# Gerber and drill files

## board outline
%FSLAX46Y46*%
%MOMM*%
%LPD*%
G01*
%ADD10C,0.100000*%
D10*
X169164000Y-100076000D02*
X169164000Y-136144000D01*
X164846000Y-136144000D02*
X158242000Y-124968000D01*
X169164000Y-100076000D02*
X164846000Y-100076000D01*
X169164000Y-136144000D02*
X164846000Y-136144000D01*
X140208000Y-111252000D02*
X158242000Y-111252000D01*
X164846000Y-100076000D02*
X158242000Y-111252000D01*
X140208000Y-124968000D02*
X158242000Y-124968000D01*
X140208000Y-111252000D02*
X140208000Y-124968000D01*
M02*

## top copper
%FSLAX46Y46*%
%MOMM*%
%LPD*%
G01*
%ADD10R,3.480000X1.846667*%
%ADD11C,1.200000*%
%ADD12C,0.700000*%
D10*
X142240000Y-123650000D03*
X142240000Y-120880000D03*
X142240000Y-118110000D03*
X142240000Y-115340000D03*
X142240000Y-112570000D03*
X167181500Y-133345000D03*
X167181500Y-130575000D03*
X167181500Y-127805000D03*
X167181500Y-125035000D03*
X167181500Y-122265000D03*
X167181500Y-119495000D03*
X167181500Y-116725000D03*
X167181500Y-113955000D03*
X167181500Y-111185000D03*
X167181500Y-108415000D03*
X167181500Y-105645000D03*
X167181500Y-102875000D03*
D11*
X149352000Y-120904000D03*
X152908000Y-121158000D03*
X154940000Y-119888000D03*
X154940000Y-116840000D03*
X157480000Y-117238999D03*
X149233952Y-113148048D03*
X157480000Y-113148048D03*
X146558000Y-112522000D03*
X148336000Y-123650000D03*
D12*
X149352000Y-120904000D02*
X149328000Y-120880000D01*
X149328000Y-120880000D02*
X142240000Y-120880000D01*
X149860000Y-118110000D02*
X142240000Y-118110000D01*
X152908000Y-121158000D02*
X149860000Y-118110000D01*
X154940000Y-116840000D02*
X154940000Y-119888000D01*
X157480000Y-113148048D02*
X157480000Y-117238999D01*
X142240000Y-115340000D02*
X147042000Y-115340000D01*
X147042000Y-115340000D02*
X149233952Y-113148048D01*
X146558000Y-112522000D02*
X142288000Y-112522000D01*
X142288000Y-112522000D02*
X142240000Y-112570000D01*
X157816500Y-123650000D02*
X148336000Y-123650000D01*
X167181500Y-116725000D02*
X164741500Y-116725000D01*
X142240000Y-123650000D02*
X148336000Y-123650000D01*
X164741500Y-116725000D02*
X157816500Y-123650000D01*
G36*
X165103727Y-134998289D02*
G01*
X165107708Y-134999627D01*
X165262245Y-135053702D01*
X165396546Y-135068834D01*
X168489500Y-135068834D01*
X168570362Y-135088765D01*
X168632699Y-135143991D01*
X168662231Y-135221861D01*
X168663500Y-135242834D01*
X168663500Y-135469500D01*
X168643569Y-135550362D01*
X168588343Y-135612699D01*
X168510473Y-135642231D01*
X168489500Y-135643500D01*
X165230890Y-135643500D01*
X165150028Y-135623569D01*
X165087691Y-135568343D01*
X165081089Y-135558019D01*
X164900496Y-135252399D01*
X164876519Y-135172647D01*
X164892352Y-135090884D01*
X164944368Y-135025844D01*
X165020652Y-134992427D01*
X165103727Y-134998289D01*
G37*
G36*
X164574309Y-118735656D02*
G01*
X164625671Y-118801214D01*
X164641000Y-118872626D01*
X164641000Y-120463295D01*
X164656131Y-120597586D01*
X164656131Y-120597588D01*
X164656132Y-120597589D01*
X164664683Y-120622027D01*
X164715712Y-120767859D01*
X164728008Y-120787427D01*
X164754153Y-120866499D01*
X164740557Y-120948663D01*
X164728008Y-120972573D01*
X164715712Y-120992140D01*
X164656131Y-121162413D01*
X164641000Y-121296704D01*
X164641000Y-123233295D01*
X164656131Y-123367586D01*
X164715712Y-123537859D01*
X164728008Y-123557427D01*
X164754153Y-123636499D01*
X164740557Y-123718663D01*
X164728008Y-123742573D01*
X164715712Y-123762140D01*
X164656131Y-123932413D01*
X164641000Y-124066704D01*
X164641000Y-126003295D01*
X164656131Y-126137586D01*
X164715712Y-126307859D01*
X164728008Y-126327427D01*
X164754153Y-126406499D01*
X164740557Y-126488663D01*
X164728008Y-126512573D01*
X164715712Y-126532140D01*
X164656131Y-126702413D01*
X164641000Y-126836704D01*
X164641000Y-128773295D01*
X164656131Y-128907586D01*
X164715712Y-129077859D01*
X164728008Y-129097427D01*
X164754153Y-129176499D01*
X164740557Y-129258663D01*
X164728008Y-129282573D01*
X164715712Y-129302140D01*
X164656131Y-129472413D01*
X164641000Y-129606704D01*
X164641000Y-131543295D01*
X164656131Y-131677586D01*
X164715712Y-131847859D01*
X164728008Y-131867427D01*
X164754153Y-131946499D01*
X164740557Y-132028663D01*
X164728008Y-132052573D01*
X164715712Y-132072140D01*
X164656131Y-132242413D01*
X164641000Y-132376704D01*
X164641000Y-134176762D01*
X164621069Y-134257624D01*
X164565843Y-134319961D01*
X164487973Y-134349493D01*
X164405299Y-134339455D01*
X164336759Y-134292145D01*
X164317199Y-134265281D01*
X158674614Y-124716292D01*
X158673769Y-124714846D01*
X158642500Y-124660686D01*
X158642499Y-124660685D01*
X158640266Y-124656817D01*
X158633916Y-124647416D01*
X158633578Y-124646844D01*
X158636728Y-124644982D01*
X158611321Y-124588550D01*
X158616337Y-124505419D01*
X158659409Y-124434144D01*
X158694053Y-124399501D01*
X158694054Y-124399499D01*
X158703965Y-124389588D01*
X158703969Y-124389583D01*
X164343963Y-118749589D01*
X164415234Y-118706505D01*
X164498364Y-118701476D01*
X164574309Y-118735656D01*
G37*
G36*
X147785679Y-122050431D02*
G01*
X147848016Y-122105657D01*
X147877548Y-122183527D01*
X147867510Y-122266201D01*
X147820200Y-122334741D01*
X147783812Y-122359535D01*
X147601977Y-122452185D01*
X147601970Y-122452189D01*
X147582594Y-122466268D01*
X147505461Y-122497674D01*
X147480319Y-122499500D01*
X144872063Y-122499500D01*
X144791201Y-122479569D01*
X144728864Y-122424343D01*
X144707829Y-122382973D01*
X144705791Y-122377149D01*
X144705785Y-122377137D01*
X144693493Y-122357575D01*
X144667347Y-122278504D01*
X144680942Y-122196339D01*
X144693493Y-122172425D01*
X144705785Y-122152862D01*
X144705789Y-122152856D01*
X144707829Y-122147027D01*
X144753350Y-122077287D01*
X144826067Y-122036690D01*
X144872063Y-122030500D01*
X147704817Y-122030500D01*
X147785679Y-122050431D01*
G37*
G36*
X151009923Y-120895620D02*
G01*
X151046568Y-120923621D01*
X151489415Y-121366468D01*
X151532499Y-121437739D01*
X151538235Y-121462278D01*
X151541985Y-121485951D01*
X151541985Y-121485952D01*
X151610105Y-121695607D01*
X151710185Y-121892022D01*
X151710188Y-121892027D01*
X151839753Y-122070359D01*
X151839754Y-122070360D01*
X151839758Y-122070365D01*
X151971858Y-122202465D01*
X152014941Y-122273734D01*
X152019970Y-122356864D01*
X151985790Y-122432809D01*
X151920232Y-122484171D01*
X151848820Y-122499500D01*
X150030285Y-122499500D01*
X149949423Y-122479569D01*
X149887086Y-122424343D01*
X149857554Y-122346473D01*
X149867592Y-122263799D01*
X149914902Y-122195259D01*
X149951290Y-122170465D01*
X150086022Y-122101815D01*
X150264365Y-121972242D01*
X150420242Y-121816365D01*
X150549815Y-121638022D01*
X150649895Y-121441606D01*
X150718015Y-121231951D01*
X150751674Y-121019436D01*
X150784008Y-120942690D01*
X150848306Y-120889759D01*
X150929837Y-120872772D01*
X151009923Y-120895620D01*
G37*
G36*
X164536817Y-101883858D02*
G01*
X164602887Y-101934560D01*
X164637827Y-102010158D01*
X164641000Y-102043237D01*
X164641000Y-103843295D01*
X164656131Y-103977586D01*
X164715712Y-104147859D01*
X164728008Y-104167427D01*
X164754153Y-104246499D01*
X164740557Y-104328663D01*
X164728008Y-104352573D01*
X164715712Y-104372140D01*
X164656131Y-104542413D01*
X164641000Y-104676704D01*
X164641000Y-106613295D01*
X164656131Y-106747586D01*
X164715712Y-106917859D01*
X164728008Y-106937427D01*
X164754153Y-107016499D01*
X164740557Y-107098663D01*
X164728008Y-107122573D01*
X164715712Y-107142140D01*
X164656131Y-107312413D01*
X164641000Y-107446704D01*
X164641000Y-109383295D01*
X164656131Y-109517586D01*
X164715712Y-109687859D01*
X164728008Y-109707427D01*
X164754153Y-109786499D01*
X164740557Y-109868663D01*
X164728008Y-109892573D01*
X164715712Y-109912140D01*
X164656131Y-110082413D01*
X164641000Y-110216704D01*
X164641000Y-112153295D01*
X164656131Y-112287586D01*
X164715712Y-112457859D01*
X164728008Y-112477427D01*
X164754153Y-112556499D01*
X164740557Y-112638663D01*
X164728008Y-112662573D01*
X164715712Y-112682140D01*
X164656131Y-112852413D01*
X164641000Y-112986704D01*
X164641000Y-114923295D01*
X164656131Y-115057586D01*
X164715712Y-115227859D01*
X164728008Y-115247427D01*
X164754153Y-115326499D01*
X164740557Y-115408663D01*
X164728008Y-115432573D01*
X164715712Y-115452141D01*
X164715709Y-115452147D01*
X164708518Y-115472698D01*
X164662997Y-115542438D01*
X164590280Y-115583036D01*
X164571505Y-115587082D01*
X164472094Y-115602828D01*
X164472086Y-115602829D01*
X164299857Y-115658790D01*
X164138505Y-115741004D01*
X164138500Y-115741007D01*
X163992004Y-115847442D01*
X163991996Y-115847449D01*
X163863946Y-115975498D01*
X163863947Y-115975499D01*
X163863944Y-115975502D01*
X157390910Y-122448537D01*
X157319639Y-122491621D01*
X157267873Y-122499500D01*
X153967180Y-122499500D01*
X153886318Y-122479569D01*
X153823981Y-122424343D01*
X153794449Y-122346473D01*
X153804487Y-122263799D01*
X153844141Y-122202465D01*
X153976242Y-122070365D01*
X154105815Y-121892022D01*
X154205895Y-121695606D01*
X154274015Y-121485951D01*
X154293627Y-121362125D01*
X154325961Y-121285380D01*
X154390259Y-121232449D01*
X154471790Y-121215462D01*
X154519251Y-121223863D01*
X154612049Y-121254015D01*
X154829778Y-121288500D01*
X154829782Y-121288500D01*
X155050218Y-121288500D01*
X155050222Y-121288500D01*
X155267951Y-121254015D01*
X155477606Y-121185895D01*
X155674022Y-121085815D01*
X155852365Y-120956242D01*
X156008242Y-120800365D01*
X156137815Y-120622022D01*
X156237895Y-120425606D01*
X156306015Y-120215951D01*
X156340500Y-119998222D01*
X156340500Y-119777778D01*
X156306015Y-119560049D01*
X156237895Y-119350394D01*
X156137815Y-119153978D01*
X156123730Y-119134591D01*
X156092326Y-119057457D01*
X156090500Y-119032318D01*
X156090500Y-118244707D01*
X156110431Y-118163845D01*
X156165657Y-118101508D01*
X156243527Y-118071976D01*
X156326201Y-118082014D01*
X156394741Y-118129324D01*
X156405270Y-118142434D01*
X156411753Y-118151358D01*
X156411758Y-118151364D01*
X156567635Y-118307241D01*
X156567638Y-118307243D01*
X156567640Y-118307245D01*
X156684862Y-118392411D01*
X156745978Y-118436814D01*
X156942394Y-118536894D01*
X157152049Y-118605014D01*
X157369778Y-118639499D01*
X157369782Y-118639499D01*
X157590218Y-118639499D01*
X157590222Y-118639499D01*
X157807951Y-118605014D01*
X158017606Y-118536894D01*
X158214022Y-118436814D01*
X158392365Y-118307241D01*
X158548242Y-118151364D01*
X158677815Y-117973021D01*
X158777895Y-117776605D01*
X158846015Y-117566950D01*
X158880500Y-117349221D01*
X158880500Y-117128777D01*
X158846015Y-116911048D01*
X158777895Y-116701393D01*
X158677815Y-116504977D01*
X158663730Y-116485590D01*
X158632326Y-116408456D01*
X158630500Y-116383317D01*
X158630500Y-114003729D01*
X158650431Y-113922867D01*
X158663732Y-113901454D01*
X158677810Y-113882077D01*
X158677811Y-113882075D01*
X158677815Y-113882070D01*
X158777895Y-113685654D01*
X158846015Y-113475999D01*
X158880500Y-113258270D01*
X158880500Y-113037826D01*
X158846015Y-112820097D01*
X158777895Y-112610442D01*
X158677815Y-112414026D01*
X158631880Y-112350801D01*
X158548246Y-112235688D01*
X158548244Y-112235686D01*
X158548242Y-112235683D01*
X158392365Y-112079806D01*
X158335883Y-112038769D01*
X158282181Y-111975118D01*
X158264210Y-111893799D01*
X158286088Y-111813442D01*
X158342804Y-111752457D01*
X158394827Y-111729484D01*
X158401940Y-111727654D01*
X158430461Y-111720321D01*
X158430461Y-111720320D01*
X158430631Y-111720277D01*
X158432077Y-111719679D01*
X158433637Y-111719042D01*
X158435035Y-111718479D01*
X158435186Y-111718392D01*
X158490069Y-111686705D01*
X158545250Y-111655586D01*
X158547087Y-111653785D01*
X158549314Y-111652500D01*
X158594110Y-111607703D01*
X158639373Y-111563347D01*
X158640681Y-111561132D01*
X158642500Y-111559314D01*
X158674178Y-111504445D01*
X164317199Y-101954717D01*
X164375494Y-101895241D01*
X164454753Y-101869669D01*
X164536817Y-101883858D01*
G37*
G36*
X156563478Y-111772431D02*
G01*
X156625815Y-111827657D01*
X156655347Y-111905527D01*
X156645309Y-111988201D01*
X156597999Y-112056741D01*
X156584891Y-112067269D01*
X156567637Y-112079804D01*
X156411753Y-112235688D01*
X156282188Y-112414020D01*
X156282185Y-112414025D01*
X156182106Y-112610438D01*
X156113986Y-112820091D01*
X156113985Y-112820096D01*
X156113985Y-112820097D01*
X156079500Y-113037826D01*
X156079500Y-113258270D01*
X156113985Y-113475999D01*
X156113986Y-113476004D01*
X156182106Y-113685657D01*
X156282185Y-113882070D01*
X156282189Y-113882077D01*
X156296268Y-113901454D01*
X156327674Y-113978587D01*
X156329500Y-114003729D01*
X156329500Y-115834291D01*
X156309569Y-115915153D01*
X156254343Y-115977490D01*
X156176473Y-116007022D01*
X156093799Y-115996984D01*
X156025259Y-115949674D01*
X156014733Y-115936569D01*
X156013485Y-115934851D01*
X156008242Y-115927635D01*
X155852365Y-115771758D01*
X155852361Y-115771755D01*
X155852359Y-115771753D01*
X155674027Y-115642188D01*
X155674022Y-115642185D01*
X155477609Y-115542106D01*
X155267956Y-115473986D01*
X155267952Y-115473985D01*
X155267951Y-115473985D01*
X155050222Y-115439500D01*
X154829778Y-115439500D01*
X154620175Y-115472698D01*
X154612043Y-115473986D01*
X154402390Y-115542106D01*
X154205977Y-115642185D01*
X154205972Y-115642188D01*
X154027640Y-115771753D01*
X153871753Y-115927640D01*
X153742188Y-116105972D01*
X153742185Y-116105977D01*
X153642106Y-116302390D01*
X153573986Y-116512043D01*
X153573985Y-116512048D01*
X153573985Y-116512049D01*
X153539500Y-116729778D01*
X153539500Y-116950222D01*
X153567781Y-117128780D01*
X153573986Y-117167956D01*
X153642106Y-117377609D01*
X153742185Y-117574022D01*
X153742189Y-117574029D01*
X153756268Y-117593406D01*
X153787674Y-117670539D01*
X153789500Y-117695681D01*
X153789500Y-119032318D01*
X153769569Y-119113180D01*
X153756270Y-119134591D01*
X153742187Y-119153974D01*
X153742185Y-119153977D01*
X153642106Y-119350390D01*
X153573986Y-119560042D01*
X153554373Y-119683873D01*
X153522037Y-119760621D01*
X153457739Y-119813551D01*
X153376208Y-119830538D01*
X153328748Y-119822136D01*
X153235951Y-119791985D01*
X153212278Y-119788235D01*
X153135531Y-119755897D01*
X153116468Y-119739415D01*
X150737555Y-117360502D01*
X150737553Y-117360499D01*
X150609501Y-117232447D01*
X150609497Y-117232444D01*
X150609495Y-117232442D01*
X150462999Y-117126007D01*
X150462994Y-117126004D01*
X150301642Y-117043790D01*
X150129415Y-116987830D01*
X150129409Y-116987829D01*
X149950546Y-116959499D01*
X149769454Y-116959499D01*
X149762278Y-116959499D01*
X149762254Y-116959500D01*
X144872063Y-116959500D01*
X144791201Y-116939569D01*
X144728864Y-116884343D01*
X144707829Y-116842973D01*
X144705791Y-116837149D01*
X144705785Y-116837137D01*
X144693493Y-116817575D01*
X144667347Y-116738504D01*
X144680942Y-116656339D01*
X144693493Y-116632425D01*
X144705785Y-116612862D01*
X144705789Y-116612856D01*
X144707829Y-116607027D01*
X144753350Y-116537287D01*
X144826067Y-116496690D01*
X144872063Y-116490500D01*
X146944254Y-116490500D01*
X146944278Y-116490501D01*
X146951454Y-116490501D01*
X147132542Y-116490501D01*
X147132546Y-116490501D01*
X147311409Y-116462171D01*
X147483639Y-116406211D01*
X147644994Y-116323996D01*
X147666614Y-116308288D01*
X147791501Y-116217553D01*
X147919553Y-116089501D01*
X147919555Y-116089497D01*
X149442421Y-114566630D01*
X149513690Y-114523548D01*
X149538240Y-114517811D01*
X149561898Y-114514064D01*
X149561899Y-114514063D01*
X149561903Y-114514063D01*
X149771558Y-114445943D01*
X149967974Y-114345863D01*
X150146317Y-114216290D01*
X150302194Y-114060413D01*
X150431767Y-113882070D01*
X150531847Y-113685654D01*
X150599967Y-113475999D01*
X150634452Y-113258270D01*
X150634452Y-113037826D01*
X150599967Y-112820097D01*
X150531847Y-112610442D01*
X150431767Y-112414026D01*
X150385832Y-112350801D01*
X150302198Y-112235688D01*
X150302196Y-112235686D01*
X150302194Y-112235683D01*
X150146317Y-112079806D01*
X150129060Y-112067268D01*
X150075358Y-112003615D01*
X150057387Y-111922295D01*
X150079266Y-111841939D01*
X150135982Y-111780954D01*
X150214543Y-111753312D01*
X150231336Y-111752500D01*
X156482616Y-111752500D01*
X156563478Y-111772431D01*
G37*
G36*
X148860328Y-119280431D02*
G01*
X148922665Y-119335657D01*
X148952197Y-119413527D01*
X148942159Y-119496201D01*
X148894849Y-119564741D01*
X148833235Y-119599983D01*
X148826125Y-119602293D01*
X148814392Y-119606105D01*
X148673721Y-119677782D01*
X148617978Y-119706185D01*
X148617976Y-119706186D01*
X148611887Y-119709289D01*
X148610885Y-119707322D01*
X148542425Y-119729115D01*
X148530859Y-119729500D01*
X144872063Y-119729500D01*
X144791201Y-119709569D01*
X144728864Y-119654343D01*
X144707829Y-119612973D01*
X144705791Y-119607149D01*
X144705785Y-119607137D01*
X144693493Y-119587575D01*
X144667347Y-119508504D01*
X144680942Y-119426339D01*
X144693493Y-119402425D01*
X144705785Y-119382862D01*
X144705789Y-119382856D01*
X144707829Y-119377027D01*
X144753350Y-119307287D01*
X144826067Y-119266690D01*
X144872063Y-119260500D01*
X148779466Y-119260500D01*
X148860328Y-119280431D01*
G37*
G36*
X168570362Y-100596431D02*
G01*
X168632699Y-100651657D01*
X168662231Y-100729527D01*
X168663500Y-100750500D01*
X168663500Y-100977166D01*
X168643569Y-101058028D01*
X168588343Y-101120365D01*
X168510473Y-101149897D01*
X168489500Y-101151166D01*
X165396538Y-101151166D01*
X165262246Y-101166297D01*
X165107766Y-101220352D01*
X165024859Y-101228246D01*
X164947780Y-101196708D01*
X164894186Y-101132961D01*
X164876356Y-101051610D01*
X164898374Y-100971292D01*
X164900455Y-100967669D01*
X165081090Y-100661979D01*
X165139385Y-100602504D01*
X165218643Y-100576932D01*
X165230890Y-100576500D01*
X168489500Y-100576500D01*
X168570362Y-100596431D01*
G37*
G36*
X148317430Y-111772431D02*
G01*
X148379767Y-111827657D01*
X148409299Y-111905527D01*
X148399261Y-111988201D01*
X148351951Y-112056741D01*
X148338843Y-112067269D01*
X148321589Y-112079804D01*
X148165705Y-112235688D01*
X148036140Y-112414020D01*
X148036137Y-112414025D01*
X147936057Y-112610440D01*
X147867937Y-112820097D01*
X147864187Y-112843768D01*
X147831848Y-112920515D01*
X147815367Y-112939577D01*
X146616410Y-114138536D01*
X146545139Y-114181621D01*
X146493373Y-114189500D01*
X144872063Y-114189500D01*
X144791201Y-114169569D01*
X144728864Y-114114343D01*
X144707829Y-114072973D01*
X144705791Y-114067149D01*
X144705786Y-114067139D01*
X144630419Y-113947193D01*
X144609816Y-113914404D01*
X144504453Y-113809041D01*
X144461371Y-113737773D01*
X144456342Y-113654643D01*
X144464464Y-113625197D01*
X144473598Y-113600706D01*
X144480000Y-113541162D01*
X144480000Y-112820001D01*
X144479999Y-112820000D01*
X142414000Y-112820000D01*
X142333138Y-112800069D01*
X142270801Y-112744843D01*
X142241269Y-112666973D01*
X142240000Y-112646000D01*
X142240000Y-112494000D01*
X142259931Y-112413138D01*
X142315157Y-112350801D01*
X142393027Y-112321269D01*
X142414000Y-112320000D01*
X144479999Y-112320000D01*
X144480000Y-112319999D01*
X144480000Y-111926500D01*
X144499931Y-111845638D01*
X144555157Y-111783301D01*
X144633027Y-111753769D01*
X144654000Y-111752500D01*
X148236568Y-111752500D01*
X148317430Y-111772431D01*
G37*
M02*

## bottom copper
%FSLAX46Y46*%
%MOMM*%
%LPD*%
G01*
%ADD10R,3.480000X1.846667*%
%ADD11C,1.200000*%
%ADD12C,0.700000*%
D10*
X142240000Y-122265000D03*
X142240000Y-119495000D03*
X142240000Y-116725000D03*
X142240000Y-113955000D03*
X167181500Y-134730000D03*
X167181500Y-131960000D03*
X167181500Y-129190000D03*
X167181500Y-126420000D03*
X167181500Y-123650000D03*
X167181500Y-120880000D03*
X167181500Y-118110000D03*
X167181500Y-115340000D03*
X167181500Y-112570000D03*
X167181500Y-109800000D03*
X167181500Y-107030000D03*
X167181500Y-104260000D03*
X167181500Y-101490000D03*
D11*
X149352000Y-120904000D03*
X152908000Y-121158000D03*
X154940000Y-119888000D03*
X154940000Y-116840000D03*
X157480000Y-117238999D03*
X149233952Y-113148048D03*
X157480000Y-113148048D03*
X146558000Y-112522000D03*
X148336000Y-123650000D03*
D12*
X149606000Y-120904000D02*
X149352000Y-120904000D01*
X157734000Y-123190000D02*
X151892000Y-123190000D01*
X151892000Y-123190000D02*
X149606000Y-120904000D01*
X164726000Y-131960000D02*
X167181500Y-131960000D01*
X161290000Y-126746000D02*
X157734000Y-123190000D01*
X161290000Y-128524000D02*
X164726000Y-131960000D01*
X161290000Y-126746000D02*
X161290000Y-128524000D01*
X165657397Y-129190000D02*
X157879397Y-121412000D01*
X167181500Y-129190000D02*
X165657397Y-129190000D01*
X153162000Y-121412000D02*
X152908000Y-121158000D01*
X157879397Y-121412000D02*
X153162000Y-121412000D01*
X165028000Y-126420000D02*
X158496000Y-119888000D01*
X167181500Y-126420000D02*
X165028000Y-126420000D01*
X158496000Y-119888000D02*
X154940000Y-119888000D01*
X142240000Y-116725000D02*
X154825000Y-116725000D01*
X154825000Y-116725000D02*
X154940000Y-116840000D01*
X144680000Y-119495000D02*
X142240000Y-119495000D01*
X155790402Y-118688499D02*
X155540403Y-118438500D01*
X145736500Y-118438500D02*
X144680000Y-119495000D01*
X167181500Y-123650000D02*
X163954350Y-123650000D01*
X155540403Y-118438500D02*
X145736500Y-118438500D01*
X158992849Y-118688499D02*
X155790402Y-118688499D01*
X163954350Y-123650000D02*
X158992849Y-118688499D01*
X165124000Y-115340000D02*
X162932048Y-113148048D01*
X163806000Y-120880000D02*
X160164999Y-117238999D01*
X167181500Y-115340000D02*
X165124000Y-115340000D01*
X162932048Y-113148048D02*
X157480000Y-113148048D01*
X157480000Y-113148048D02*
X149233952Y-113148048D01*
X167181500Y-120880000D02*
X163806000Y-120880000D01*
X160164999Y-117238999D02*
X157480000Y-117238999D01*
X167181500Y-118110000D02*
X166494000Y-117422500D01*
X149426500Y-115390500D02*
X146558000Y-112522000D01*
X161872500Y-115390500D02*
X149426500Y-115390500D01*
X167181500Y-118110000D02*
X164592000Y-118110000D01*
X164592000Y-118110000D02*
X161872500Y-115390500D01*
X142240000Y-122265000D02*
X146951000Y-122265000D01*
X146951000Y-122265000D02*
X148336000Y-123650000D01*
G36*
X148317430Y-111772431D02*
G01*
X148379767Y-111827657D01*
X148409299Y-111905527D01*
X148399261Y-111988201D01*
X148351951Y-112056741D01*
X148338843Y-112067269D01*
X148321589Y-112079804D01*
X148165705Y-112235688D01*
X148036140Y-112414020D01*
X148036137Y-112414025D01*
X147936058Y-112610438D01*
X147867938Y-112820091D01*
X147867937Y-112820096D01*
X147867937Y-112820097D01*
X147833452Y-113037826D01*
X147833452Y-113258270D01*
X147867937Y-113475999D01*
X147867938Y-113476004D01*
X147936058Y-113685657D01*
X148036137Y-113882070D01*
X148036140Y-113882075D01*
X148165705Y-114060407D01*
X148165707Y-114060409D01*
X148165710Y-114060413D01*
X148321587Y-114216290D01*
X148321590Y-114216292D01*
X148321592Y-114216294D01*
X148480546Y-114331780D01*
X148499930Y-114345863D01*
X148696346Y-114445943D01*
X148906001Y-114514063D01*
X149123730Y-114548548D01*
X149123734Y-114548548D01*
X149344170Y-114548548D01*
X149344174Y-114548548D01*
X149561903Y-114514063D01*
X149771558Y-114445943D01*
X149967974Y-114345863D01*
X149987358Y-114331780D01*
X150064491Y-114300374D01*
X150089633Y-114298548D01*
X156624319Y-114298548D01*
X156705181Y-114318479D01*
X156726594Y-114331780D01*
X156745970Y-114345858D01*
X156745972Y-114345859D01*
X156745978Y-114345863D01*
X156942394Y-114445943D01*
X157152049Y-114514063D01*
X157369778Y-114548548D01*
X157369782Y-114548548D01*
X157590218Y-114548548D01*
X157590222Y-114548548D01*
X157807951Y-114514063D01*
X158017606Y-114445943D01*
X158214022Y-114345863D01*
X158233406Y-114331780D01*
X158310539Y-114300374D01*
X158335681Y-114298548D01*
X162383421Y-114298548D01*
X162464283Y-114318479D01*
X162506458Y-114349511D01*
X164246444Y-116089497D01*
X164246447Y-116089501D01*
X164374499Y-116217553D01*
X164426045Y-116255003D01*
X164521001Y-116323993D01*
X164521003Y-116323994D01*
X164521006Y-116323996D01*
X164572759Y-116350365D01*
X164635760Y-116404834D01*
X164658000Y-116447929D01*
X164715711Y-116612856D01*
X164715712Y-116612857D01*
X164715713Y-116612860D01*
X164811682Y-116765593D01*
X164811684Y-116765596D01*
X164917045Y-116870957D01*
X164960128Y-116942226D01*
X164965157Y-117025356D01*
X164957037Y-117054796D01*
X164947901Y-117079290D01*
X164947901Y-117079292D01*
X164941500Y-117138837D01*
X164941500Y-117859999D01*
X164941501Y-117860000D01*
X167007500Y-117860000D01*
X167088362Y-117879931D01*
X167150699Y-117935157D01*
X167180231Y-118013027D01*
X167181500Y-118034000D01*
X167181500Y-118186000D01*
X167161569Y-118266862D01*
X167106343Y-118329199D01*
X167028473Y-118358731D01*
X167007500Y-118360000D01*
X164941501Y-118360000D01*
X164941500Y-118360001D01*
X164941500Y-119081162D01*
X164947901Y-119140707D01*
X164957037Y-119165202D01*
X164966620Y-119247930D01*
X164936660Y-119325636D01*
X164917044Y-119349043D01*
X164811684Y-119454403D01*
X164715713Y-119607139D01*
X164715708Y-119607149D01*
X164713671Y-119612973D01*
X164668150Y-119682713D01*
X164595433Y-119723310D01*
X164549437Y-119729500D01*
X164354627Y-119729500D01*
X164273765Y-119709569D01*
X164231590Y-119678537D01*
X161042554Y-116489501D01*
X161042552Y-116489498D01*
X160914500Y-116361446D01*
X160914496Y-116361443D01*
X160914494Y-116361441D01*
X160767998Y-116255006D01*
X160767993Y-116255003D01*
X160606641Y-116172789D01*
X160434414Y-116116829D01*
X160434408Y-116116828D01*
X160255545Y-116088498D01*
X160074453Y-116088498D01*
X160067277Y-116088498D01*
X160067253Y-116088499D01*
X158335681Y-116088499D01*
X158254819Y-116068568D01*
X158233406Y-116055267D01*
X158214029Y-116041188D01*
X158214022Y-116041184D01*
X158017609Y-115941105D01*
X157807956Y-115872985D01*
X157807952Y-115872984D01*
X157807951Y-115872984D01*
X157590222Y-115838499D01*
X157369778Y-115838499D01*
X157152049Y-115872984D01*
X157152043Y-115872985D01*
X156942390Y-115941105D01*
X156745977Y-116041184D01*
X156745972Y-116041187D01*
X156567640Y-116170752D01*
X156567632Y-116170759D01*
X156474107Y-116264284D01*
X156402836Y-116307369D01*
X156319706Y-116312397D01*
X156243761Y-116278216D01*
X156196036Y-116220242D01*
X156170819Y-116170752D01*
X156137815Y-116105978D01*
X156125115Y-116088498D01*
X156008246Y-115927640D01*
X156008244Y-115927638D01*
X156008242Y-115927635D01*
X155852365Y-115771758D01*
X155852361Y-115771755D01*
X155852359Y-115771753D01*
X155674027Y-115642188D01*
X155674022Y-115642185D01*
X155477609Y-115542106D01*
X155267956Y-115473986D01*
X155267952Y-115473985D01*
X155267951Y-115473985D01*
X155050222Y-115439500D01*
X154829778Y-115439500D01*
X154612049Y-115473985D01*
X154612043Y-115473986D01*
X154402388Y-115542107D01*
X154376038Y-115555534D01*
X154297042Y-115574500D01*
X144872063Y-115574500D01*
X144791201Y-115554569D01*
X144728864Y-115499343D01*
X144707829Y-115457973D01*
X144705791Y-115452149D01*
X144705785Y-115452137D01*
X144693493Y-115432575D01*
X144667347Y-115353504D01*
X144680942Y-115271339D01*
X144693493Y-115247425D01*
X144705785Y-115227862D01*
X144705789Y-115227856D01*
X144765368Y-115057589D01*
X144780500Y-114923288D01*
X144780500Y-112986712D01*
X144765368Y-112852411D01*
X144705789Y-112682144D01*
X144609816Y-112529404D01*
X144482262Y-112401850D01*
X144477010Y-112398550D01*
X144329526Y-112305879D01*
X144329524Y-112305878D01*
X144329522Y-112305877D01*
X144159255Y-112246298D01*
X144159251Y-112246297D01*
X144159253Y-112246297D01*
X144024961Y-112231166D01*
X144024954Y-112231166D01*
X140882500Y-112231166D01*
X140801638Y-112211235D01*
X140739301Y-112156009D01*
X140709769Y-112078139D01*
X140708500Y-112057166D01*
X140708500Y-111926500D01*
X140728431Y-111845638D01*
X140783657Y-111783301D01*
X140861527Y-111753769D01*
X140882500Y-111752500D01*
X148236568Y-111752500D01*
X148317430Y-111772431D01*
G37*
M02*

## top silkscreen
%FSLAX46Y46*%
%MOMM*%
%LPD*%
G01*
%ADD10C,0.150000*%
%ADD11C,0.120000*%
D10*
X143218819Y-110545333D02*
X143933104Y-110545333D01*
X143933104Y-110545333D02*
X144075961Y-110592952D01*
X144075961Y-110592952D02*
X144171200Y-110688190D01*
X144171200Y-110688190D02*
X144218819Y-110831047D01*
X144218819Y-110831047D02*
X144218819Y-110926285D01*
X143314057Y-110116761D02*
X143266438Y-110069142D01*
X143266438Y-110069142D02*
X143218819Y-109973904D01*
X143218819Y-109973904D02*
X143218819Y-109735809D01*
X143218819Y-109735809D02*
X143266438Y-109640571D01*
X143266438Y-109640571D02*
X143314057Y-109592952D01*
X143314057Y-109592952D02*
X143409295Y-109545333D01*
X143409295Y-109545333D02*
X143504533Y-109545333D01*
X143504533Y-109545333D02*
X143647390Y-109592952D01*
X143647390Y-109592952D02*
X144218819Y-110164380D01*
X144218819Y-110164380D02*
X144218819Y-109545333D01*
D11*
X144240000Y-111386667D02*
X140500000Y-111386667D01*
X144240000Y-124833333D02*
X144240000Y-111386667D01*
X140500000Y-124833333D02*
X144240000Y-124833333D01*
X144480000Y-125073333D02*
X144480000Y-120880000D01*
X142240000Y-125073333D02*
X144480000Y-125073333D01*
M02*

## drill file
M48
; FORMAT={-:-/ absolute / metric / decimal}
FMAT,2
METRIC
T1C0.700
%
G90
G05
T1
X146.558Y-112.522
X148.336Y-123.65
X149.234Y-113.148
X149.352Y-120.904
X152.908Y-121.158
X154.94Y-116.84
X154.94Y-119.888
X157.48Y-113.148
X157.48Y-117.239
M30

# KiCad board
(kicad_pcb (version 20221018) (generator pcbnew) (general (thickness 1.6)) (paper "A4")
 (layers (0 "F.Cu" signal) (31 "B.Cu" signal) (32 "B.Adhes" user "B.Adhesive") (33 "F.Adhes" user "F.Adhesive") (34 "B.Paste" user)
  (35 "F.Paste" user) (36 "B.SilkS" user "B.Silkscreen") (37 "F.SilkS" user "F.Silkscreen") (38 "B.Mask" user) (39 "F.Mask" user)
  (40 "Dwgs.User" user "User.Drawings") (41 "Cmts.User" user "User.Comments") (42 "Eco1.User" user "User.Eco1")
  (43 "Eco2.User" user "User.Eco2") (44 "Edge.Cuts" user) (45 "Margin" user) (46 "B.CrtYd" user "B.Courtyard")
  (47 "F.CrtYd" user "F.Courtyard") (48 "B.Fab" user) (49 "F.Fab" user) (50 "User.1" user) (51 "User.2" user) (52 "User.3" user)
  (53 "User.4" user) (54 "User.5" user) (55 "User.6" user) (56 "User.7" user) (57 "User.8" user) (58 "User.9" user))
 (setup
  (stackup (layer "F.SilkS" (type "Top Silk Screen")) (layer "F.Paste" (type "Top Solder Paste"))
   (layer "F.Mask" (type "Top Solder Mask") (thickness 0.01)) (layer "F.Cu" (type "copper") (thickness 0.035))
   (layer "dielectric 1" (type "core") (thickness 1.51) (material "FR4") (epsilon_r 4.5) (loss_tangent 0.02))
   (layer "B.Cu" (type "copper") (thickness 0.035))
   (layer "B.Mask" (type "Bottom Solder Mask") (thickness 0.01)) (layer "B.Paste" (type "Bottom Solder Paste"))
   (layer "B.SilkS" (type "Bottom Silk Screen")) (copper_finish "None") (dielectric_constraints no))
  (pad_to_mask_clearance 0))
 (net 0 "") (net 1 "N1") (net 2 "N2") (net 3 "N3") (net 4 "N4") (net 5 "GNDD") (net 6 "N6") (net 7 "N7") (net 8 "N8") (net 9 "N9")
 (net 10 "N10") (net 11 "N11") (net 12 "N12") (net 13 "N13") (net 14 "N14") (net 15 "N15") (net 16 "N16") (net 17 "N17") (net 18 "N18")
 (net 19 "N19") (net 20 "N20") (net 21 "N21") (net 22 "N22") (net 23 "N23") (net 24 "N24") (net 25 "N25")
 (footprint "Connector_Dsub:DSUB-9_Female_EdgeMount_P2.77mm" (layer "F.Cu") (at 142.24 118.11 -90)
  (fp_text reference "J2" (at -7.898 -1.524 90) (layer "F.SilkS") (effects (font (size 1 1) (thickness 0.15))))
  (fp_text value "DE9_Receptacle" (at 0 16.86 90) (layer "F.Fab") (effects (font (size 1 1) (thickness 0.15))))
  (fp_line (start -6.723333 -2) (end -6.723333 1.74) (stroke (width 0.12) (type solid)) (layer "F.SilkS"))
  (fp_line (start 6.723333 -2) (end -6.723333 -2) (stroke (width 0.12) (type solid)) (layer "F.SilkS"))
  (fp_line (start 6.723333 1.74) (end 6.723333 -2) (stroke (width 0.12) (type solid)) (layer "F.SilkS"))
  (fp_line (start 6.963333 -2.24) (end 2.77 -2.24) (stroke (width 0.12) (type solid)) (layer "F.SilkS"))
  (fp_line (start 6.963333 0) (end 6.963333 -2.24) (stroke (width 0.12) (type solid)) (layer "F.SilkS"))
  (pad "1" smd rect (at 5.54 0 270) (size 1.846667 3.48) (layers "F.Cu" "F.Paste" "F.Mask") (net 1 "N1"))
  (pad "2" smd rect (at 2.77 0 270) (size 1.846667 3.48) (layers "F.Cu" "F.Paste" "F.Mask") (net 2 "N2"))
  (pad "3" smd rect (at 0 0 270) (size 1.846667 3.48) (layers "F.Cu" "F.Paste" "F.Mask") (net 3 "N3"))
  (pad "4" smd rect (at -2.77 0 270) (size 1.846667 3.48) (layers "F.Cu" "F.Paste" "F.Mask") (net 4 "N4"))
  (pad "5" smd rect (at -5.54 0 270) (size 1.846667 3.48) (layers "F.Cu" "F.Paste" "F.Mask") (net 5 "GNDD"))
  (pad "6" smd rect (at 4.155 0 270) (size 1.846667 3.48) (layers "B.Cu" "B.Paste" "B.Mask") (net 1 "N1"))
  (pad "7" smd rect (at 1.385 0 270) (size 1.846667 3.48) (layers "B.Cu" "B.Paste" "B.Mask") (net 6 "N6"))
  (pad "8" smd rect (at -1.385 0 270) (size 1.846667 3.48) (layers "B.Cu" "B.Paste" "B.Mask") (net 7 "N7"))
  (pad "9" smd rect (at -4.155 0 270) (size 1.846667 3.48) (layers "B.Cu" "B.Paste" "B.Mask") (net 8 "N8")))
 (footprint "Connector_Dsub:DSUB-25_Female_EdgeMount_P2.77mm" (layer "B.Cu") (at 167.1815 118.11 -90)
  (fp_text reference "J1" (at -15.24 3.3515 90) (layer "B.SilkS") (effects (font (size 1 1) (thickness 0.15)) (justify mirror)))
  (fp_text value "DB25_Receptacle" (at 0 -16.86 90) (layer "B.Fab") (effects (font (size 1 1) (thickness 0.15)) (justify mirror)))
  (pad "1" smd rect (at 16.62 0 270) (size 1.846667 3.48) (layers "B.Cu" "B.Paste" "B.Mask") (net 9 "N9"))
  (pad "2" smd rect (at 13.85 0 270) (size 1.846667 3.48) (layers "B.Cu" "B.Paste" "B.Mask") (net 2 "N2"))
  (pad "3" smd rect (at 11.08 0 270) (size 1.846667 3.48) (layers "B.Cu" "B.Paste" "B.Mask") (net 3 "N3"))
  (pad "4" smd rect (at 8.31 0 270) (size 1.846667 3.48) (layers "B.Cu" "B.Paste" "B.Mask") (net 7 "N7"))
  (pad "5" smd rect (at 5.54 0 270) (size 1.846667 3.48) (layers "B.Cu" "B.Paste" "B.Mask") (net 6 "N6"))
  (pad "6" smd rect (at 2.77 0 270) (size 1.846667 3.48) (layers "B.Cu" "B.Paste" "B.Mask") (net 4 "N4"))
  (pad "7" smd rect (at 0 0 270) (size 1.846667 3.48) (layers "B.Cu" "B.Paste" "B.Mask") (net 5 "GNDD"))
  (pad "8" smd rect (at -2.77 0 270) (size 1.846667 3.48) (layers "B.Cu" "B.Paste" "B.Mask") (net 4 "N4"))
  (pad "9" smd rect (at -5.54 0 270) (size 1.846667 3.48) (layers "B.Cu" "B.Paste" "B.Mask") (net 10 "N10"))
  (pad "10" smd rect (at -8.31 0 270) (size 1.846667 3.48) (layers "B.Cu" "B.Paste" "B.Mask") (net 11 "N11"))
  (pad "11" smd rect (at -11.08 0 270) (size 1.846667 3.48) (layers "B.Cu" "B.Paste" "B.Mask") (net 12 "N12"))
  (pad "12" smd rect (at -13.85 0 270) (size 1.846667 3.48) (layers "B.Cu" "B.Paste" "B.Mask") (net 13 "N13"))
  (pad "13" smd rect (at -16.62 0 270) (size 1.846667 3.48) (layers "B.Cu" "B.Paste" "B.Mask") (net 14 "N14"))
  (pad "14" smd rect (at 15.235 0 270) (size 1.846667 3.48) (layers "F.Cu" "F.Paste" "F.Mask") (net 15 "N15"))
  (pad "15" smd rect (at 12.465 0 270) (size 1.846667 3.48) (layers "F.Cu" "F.Paste" "F.Mask") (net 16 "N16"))
  (pad "16" smd rect (at 9.695 0 270) (size 1.846667 3.48) (layers "F.Cu" "F.Paste" "F.Mask") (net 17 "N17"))
  (pad "17" smd rect (at 6.925 0 270) (size 1.846667 3.48) (layers "F.Cu" "F.Paste" "F.Mask") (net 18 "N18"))
  (pad "18" smd rect (at 4.155 0 270) (size 1.846667 3.48) (layers "F.Cu" "F.Paste" "F.Mask") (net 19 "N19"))
  (pad "19" smd rect (at 1.385 0 270) (size 1.846667 3.48) (layers "F.Cu" "F.Paste" "F.Mask") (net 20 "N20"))
  (pad "20" smd rect (at -1.385 0 270) (size 1.846667 3.48) (layers "F.Cu" "F.Paste" "F.Mask") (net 1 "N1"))
  (pad "21" smd rect (at -4.155 0 270) (size 1.846667 3.48) (layers "F.Cu" "F.Paste" "F.Mask") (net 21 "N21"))
  (pad "22" smd rect (at -6.925 0 270) (size 1.846667 3.48) (layers "F.Cu" "F.Paste" "F.Mask") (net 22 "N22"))
  (pad "23" smd rect (at -9.695 0 270) (size 1.846667 3.48) (layers "F.Cu" "F.Paste" "F.Mask") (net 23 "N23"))
  (pad "24" smd rect (at -12.465 0 270) (size 1.846667 3.48) (layers "F.Cu" "F.Paste" "F.Mask") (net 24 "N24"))
  (pad "25" smd rect (at -15.235 0 270) (size 1.846667 3.48) (layers "F.Cu" "F.Paste" "F.Mask") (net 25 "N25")))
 (gr_line (start 169.164 100.076) (end 169.164 136.144) (stroke (width 0.1) (type default)) (layer "Edge.Cuts"))
 (gr_line (start 164.846 136.144) (end 158.242 124.968) (stroke (width 0.1) (type default)) (layer "Edge.Cuts"))
 (gr_line (start 169.164 100.076) (end 164.846 100.076) (stroke (width 0.1) (type default)) (layer "Edge.Cuts"))
 (gr_line (start 169.164 136.144) (end 164.846 136.144) (stroke (width 0.1) (type default)) (layer "Edge.Cuts"))
 (gr_line (start 140.208 111.252) (end 158.242 111.252) (stroke (width 0.1) (type default)) (layer "Edge.Cuts"))
 (gr_line (start 164.846 100.076) (end 158.242 111.252) (stroke (width 0.1) (type default)) (layer "Edge.Cuts"))
 (gr_line (start 140.208 124.968) (end 158.242 124.968) (stroke (width 0.1) (type default)) (layer "Edge.Cuts"))
 (gr_line (start 140.208 111.252) (end 140.208 124.968) (stroke (width 0.1) (type default)) (layer "Edge.Cuts"))
 (segment (start 149.352 120.904) (end 149.328 120.88) (width 0.7) (layer "F.Cu") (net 2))
 (segment (start 149.328 120.88) (end 142.24 120.88) (width 0.7) (layer "F.Cu") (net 2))
 (via (at 149.352 120.904) (size 1.2) (drill 0.7) (layers "F.Cu" "B.Cu") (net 2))
 (segment (start 149.606 120.904) (end 149.352 120.904) (width 0.7) (layer "B.Cu") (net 2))
 (segment (start 157.734 123.19) (end 151.892 123.19) (width 0.7) (layer "B.Cu") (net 2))
 (segment (start 151.892 123.19) (end 149.606 120.904) (width 0.7) (layer "B.Cu") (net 2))
 (segment (start 164.726 131.96) (end 167.1815 131.96) (width 0.7) (layer "B.Cu") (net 2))
 (segment (start 161.29 126.746) (end 157.734 123.19) (width 0.7) (layer "B.Cu") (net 2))
 (segment (start 161.29 128.524) (end 164.726 131.96) (width 0.7) (layer "B.Cu") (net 2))
 (segment (start 161.29 126.746) (end 161.29 128.524) (width 0.7) (layer "B.Cu") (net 2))
 (segment (start 149.86 118.11) (end 142.24 118.11) (width 0.7) (layer "F.Cu") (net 3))
 (segment (start 152.908 121.158) (end 149.86 118.11) (width 0.7) (layer "F.Cu") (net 3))
 (via (at 152.908 121.158) (size 1.2) (drill 0.7) (layers "F.Cu" "B.Cu") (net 3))
 (segment (start 165.657397 129.19) (end 157.879397 121.412) (width 0.7) (layer "B.Cu") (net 3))
 (segment (start 167.1815 129.19) (end 165.657397 129.19) (width 0.7) (layer "B.Cu") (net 3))
 (segment (start 153.162 121.412) (end 152.908 121.158) (width 0.7) (layer "B.Cu") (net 3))
 (segment (start 157.879397 121.412) (end 153.162 121.412) (width 0.7) (layer "B.Cu") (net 3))
 (segment (start 154.94 116.84) (end 154.94 119.888) (width 0.7) (layer "F.Cu") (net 7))
 (via (at 154.94 119.888) (size 1.2) (drill 0.7) (layers "F.Cu" "B.Cu") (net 7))
 (via (at 154.94 116.84) (size 1.2) (drill 0.7) (layers "F.Cu" "B.Cu") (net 7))
 (segment (start 165.028 126.42) (end 158.496 119.888) (width 0.7) (layer "B.Cu") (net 7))
 (segment (start 167.1815 126.42) (end 165.028 126.42) (width 0.7) (layer "B.Cu") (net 7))
 (segment (start 158.496 119.888) (end 154.94 119.888) (width 0.7) (layer "B.Cu") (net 7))
 (segment (start 142.24 116.725) (end 154.825 116.725) (width 0.7) (layer "B.Cu") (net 7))
 (segment (start 154.825 116.725) (end 154.94 116.84) (width 0.7) (layer "B.Cu") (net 7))
 (segment (start 144.68 119.495) (end 142.24 119.495) (width 0.7) (layer "B.Cu") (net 6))
 (segment (start 155.790402 118.688499) (end 155.540403 118.4385) (width 0.7) (layer "B.Cu") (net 6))
 (segment (start 145.7365 118.4385) (end 144.68 119.495) (width 0.7) (layer "B.Cu") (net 6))
 (segment (start 167.1815 123.65) (end 163.95435 123.65) (width 0.7) (layer "B.Cu") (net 6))
 (segment (start 155.540403 118.4385) (end 145.7365 118.4385) (width 0.7) (layer "B.Cu") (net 6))
 (segment (start 158.992849 118.688499) (end 155.790402 118.688499) (width 0.7) (layer "B.Cu") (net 6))
 (segment (start 163.95435 123.65) (end 158.992849 118.688499) (width 0.7) (layer "B.Cu") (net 6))
 (segment (start 157.48 113.148048) (end 157.48 117.238999) (width 0.7) (layer "F.Cu") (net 4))
 (segment (start 142.24 115.34) (end 147.042 115.34) (width 0.7) (layer "F.Cu") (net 4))
 (segment (start 147.042 115.34) (end 149.233952 113.148048) (width 0.7) (layer "F.Cu") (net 4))
 (via (at 157.48 117.238999) (size 1.2) (drill 0.7) (layers "F.Cu" "B.Cu") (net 4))
 (via (at 149.233952 113.148048) (size 1.2) (drill 0.7) (layers "F.Cu" "B.Cu") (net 4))
 (via (at 157.48 113.148048) (size 1.2) (drill 0.7) (layers "F.Cu" "B.Cu") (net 4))
 (segment (start 165.124 115.34) (end 162.932048 113.148048) (width 0.7) (layer "B.Cu") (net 4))
 (segment (start 163.806 120.88) (end 160.164999 117.238999) (width 0.7) (layer "B.Cu") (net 4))
 (segment (start 167.1815 115.34) (end 165.124 115.34) (width 0.7) (layer "B.Cu") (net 4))
 (segment (start 162.932048 113.148048) (end 157.48 113.148048) (width 0.7) (layer "B.Cu") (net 4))
 (segment (start 157.48 113.148048) (end 149.233952 113.148048) (width 0.7) (layer "B.Cu") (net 4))
 (segment (start 167.1815 120.88) (end 163.806 120.88) (width 0.7) (layer "B.Cu") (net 4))
 (segment (start 160.164999 117.238999) (end 157.48 117.238999) (width 0.7) (layer "B.Cu") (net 4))
 (segment (start 146.558 112.522) (end 142.288 112.522) (width 0.7) (layer "F.Cu") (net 5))
 (segment (start 142.288 112.522) (end 142.24 112.57) (width 0.7) (layer "F.Cu") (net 5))
 (via (at 146.558 112.522) (size 1.2) (drill 0.7) (layers "F.Cu" "B.Cu") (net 5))
 (segment (start 167.1815 118.11) (end 166.494 117.4225) (width 0.7) (layer "B.Cu") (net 5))
 (segment (start 149.4265 115.3905) (end 146.558 112.522) (width 0.7) (layer "B.Cu") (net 5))
 (segment (start 161.8725 115.3905) (end 149.4265 115.3905) (width 0.7) (layer "B.Cu") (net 5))
 (segment (start 167.1815 118.11) (end 164.592 118.11) (width 0.7) (layer "B.Cu") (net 5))
 (segment (start 164.592 118.11) (end 161.8725 115.3905) (width 0.7) (layer "B.Cu") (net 5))
 (segment (start 157.8165 123.65) (end 148.336 123.65) (width 0.7) (layer "F.Cu") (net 1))
 (segment (start 167.1815 116.725) (end 164.7415 116.725) (width 0.7) (layer "F.Cu") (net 1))
 (segment (start 142.24 123.65) (end 148.336 123.65) (width 0.7) (layer "F.Cu") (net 1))
 (segment (start 164.7415 116.725) (end 157.8165 123.65) (width 0.7) (layer "F.Cu") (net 1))
 (via (at 148.336 123.65) (size 1.2) (drill 0.7) (layers "F.Cu" "B.Cu") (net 1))
 (segment (start 142.24 122.265) (end 146.951 122.265) (width 0.7) (layer "B.Cu") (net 1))
 (segment (start 146.951 122.265) (end 148.336 123.65) (width 0.7) (layer "B.Cu") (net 1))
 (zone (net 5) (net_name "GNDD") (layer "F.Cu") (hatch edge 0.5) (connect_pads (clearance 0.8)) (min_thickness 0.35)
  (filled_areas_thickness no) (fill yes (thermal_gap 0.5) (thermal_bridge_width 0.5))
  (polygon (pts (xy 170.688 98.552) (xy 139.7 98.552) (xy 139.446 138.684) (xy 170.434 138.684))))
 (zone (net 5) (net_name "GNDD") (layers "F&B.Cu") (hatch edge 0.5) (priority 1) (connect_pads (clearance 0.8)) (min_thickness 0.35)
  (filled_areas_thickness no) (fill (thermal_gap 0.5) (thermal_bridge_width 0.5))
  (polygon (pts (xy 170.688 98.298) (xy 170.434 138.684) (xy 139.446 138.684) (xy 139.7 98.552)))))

